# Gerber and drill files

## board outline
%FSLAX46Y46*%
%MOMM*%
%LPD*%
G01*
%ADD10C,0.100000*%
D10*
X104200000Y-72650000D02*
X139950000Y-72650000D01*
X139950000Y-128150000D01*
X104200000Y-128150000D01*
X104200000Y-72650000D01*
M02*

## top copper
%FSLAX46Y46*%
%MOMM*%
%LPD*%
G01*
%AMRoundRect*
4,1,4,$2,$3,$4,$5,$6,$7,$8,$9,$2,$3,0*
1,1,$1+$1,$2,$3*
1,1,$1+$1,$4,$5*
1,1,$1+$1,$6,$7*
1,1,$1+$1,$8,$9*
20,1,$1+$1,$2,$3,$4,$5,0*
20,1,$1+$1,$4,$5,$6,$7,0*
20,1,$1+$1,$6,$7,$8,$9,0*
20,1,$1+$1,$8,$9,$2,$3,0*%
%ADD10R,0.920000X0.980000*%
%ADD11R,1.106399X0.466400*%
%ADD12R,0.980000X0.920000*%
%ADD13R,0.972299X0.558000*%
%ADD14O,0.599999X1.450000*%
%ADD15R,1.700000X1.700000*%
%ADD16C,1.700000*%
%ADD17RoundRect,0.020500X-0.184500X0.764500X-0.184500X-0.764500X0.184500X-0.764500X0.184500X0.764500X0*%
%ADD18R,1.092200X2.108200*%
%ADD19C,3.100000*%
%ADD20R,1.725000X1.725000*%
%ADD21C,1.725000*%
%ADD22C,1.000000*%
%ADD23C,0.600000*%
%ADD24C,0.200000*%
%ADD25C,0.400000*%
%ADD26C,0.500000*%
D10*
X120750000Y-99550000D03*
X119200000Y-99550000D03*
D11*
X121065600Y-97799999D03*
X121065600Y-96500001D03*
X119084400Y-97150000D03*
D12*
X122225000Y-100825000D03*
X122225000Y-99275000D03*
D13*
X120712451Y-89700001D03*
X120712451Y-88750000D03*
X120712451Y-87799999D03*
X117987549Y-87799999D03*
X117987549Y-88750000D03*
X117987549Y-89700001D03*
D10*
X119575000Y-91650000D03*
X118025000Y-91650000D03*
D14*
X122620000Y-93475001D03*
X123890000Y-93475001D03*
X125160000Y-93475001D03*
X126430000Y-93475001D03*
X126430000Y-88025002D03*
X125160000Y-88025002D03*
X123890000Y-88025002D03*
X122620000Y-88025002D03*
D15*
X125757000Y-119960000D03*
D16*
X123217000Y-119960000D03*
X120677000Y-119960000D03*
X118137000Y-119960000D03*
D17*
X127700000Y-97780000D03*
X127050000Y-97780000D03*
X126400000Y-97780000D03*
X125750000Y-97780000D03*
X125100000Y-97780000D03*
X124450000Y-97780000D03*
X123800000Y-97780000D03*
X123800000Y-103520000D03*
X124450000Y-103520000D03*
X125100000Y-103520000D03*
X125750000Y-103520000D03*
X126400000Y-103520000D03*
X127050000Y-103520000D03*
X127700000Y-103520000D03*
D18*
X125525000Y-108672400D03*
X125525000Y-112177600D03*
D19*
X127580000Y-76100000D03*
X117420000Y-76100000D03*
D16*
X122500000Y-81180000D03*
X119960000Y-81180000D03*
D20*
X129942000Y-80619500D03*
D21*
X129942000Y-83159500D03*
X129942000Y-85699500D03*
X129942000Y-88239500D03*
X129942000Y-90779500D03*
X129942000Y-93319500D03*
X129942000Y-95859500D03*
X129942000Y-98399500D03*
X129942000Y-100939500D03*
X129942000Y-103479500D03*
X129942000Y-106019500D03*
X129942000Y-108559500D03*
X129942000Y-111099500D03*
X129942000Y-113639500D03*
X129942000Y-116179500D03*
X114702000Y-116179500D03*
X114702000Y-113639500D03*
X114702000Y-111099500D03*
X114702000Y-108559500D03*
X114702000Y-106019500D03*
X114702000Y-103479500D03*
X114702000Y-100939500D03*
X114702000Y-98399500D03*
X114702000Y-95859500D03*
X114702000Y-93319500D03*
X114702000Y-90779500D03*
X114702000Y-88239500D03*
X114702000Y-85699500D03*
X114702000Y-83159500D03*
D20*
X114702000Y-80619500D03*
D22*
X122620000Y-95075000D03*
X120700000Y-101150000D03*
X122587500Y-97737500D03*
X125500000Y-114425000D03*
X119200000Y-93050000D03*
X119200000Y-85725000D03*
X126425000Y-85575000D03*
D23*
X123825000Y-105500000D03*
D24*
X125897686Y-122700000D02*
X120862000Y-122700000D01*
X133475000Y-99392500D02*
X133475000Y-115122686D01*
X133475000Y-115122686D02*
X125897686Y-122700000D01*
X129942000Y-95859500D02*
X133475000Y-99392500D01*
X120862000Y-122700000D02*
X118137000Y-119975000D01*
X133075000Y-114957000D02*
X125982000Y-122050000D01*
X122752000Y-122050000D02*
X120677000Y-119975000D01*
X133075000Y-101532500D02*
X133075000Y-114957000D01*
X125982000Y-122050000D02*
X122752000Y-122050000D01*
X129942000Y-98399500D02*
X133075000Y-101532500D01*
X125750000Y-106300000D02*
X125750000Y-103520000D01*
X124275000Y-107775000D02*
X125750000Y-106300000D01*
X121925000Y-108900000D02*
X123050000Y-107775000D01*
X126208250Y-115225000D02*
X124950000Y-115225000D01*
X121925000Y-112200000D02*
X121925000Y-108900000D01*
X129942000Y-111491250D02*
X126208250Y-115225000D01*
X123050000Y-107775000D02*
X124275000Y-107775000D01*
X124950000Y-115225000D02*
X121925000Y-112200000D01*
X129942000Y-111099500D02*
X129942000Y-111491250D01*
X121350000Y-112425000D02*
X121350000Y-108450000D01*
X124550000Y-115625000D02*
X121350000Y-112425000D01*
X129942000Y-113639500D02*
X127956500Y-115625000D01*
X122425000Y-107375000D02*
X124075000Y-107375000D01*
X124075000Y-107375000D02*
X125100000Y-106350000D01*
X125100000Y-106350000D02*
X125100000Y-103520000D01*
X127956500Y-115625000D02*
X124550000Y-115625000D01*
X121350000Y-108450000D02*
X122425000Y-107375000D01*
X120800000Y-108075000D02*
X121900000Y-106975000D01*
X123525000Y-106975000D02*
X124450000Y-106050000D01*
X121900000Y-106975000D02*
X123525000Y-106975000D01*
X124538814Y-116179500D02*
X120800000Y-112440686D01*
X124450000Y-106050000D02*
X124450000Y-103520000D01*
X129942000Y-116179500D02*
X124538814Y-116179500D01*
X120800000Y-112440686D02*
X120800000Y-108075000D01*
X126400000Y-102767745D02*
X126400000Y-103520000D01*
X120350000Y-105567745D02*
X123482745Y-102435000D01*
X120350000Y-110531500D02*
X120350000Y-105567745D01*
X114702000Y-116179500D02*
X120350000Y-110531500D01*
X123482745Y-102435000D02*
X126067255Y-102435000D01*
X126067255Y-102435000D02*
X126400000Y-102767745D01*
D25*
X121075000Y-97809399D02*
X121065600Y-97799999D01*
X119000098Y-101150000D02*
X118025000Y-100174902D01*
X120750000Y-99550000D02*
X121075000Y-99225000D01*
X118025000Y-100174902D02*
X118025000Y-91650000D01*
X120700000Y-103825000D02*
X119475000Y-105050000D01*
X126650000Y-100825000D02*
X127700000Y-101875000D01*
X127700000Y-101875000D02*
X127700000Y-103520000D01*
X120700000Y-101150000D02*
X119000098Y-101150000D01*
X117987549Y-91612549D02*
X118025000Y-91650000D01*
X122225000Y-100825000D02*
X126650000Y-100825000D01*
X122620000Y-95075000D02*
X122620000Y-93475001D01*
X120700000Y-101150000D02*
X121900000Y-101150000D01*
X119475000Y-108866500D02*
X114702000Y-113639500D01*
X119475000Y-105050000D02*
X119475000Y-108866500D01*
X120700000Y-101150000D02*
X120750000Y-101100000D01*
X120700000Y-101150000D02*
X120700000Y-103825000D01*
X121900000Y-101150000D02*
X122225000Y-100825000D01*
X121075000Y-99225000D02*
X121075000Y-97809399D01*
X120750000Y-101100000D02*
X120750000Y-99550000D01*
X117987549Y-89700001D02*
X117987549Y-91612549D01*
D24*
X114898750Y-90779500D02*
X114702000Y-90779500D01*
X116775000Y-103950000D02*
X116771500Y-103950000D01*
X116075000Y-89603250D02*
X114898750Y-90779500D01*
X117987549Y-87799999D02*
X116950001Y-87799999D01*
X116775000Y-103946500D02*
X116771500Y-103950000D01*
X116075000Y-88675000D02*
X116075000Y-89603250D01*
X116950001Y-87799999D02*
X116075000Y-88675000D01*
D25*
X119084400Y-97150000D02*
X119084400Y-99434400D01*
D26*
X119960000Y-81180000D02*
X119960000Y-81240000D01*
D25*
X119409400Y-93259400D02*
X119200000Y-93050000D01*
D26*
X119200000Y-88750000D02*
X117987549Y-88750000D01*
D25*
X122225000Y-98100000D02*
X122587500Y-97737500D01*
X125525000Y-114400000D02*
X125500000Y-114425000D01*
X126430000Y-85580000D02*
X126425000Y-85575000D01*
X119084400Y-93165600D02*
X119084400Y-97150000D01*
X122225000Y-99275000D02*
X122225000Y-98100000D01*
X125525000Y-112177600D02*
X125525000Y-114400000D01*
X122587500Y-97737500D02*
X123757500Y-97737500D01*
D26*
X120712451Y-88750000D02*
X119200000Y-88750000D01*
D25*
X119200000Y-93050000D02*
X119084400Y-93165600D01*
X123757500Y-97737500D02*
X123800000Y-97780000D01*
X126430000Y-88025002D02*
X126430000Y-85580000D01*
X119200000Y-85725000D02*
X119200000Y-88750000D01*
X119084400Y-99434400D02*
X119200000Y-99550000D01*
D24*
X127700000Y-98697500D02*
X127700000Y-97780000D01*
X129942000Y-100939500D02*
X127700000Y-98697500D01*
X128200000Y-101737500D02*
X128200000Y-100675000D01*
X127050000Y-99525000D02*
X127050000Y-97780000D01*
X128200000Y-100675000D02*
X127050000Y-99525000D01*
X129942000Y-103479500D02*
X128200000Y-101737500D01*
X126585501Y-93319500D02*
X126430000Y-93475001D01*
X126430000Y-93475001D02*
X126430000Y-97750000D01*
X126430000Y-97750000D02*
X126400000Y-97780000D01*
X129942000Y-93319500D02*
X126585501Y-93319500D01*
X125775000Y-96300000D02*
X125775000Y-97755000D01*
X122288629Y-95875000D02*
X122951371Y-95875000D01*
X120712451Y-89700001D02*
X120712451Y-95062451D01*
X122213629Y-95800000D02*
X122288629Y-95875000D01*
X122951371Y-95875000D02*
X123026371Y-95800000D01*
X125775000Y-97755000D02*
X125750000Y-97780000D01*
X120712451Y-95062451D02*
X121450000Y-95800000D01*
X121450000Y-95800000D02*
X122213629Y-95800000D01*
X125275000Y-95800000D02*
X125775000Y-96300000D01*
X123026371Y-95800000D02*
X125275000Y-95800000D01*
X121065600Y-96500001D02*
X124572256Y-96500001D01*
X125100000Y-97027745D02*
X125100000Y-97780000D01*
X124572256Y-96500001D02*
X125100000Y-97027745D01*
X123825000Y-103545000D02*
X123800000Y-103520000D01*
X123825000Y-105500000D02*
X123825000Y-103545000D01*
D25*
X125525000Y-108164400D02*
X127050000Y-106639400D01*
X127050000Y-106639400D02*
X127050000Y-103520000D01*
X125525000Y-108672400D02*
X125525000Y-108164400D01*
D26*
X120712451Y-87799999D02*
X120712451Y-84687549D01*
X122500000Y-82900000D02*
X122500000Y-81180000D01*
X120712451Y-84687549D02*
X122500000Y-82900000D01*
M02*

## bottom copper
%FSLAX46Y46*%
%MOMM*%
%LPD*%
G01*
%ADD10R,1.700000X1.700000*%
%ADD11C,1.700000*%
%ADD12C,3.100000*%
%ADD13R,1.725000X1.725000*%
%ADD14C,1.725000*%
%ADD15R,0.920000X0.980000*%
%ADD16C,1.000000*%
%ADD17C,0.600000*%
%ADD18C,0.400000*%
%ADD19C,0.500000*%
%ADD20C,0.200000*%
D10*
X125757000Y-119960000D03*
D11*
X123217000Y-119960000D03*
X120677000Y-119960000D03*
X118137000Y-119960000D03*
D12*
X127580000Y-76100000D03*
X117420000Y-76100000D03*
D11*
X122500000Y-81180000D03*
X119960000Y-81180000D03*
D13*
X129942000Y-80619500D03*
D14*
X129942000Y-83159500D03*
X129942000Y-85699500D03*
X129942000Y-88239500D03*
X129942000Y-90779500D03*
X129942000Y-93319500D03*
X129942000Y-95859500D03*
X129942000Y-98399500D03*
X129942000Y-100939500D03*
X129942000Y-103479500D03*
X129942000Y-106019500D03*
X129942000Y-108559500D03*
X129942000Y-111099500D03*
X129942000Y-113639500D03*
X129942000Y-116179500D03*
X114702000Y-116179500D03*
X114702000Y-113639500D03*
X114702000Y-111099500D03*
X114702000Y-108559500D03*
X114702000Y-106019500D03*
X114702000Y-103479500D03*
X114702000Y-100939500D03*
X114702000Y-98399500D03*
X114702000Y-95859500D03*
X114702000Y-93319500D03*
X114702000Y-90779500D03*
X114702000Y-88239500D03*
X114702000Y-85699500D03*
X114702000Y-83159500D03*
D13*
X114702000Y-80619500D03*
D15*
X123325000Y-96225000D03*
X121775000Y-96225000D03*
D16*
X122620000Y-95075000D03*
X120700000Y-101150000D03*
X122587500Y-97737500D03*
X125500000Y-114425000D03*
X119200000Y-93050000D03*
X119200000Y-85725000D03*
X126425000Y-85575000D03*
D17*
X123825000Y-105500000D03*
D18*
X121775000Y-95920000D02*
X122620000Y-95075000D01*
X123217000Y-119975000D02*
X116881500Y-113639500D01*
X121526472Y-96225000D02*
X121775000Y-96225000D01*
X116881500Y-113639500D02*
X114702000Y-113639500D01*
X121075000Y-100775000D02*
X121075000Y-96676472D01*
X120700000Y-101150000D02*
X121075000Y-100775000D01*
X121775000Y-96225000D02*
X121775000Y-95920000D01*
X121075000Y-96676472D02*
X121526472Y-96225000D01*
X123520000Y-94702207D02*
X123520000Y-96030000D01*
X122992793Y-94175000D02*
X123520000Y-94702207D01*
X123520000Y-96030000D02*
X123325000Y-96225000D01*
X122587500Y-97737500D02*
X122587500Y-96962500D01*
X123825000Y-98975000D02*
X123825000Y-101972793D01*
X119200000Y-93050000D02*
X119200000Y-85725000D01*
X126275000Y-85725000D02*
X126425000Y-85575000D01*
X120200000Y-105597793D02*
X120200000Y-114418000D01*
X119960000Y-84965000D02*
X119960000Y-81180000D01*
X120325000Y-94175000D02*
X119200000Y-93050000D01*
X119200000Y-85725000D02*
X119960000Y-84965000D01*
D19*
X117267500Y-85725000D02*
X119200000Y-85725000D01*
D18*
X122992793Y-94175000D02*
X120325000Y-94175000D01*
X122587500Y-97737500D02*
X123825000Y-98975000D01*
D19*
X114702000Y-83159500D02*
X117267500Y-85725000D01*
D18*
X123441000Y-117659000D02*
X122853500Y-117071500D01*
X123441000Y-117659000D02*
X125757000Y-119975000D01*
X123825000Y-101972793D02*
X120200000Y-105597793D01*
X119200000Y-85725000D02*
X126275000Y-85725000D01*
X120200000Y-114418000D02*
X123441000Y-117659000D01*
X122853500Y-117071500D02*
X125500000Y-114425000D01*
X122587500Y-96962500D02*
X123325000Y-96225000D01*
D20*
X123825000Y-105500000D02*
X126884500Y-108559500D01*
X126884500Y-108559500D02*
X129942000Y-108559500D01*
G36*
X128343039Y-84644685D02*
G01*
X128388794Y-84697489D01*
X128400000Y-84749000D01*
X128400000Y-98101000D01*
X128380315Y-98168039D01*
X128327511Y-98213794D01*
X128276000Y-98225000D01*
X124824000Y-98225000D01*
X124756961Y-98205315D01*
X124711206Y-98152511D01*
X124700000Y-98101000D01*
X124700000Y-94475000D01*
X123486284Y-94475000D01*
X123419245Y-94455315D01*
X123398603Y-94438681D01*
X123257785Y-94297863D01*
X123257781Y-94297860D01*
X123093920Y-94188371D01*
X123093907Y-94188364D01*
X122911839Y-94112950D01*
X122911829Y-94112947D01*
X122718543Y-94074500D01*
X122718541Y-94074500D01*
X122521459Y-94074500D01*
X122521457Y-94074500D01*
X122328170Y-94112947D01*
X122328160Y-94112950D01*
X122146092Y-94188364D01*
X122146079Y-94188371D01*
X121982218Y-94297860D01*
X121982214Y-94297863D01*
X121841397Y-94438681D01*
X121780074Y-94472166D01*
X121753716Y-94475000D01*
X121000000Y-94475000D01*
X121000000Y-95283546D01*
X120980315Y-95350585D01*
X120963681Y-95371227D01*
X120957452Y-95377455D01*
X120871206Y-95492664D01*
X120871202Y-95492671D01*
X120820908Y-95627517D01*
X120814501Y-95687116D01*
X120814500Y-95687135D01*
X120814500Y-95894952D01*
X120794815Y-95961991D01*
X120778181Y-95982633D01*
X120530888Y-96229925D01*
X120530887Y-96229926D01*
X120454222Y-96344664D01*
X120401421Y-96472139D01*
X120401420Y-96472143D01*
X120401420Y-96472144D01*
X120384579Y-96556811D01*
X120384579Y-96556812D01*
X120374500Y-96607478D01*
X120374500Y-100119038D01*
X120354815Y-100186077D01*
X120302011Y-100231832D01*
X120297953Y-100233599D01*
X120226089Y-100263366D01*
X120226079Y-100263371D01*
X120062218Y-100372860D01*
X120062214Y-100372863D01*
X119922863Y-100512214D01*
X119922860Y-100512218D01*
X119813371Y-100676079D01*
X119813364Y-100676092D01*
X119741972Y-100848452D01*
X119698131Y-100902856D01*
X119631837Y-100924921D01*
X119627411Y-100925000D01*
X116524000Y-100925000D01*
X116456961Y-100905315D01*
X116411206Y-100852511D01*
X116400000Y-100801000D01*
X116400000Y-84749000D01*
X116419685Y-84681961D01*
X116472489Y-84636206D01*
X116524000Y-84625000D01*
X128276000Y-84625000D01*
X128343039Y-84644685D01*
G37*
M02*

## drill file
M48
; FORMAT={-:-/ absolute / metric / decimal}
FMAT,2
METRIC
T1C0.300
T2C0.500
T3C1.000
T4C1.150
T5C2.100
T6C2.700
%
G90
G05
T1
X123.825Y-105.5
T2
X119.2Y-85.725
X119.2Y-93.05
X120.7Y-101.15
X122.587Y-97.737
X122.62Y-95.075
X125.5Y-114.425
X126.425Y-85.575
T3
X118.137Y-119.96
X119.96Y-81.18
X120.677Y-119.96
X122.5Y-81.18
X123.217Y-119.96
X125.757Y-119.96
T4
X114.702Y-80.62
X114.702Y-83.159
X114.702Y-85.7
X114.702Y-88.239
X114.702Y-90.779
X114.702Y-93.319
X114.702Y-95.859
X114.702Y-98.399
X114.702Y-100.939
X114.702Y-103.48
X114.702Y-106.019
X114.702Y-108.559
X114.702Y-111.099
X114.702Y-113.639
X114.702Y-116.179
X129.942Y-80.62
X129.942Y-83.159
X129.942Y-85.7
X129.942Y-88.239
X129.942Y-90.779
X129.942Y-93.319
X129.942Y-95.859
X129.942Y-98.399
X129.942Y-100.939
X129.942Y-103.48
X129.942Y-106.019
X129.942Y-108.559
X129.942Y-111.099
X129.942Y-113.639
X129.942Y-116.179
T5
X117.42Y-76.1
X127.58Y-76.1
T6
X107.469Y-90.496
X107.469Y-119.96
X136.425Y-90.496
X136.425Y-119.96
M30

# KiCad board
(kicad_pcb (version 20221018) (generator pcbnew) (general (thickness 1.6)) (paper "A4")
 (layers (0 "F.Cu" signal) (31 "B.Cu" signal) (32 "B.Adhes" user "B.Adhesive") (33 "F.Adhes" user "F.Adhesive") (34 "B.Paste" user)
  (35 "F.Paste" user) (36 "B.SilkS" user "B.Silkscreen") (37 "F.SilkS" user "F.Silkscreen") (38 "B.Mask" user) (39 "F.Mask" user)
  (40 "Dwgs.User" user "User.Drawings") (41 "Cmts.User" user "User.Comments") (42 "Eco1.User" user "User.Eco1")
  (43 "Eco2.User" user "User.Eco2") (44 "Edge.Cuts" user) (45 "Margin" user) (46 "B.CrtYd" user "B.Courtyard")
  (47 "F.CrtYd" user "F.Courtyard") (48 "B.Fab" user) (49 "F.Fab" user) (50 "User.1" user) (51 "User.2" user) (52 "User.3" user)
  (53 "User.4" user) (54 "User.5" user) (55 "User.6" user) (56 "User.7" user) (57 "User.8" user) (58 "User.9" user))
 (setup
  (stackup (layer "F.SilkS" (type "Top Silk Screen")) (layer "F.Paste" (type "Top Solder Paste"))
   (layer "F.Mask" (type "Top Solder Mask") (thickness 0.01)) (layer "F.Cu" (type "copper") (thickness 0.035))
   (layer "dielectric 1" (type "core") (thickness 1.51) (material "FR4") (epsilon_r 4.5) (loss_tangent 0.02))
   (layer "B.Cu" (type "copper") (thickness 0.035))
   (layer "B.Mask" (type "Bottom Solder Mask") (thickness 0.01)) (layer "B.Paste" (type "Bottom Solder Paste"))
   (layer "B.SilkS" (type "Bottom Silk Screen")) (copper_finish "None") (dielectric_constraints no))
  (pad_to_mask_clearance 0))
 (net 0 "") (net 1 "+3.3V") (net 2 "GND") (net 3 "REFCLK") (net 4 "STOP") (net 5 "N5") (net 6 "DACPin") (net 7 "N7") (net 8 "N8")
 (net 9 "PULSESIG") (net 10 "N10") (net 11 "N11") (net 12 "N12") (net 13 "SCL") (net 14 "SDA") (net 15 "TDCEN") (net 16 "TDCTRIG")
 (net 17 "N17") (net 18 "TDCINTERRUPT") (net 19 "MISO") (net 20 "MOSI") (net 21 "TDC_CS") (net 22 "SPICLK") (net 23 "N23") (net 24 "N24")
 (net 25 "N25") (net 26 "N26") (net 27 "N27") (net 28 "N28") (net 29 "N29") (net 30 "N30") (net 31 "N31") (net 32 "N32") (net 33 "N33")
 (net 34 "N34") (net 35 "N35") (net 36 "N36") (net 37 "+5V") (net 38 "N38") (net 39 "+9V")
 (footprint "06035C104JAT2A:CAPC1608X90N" (layer "F.Cu") (at 119.975 99.55 180)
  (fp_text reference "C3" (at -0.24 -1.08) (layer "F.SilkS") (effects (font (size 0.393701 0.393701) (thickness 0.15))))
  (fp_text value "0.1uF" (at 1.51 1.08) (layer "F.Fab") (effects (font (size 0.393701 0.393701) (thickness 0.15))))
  (pad "1" smd rect (at -0.775 0 180) (size 0.92 0.98) (layers "F.Cu" "F.Paste" "F.Mask") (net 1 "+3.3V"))
  (pad "2" smd rect (at 0.775 0 180) (size 0.92 0.98) (layers "F.Cu" "F.Paste" "F.Mask") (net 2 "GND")))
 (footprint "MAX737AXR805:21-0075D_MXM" (layer "F.Cu") (at 120.075 97.15 90)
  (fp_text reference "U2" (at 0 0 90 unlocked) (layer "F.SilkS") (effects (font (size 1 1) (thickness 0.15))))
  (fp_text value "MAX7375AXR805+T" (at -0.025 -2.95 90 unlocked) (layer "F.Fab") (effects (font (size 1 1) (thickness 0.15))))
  (pad "1" smd rect (at -0.649999 0.9906 90) (size 0.4664 1.106399) (layers "F.Cu" "F.Paste" "F.Mask") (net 1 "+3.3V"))
  (pad "2" smd rect (at 0.649999 0.9906 90) (size 0.4664 1.106399) (layers "F.Cu" "F.Paste" "F.Mask") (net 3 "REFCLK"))
  (pad "3" smd rect (at 0 -0.9906 90) (size 0.4664 1.106399) (layers "F.Cu" "F.Paste" "F.Mask") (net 2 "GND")))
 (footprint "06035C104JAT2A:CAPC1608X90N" (layer "F.Cu") (at 122.225 100.05 90)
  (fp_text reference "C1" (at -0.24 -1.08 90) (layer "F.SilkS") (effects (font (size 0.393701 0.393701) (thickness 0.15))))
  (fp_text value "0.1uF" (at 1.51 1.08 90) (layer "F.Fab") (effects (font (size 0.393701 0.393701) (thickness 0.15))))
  (pad "1" smd rect (at -0.775 0 90) (size 0.92 0.98) (layers "F.Cu" "F.Paste" "F.Mask") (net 1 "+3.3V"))
  (pad "2" smd rect (at 0.775 0 90) (size 0.92 0.98) (layers "F.Cu" "F.Paste" "F.Mask") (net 2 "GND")))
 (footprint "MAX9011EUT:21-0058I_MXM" (layer "F.Cu") (at 119.35 88.75 180)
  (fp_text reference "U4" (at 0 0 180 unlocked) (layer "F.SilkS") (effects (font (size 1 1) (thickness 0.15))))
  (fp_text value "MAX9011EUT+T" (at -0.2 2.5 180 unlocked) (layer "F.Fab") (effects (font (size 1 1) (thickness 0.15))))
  (pad "1" smd rect (at -1.362451 -0.950001 180) (size 0.972299 0.558) (layers "F.Cu" "F.Paste" "F.Mask") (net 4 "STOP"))
  (pad "2" smd rect (at -1.362451 0 180) (size 0.972299 0.558) (layers "F.Cu" "F.Paste" "F.Mask") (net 2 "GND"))
  (pad "3" smd rect (at -1.362451 0.950001 180) (size 0.972299 0.558) (layers "F.Cu" "F.Paste" "F.Mask") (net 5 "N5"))
  (pad "4" smd rect (at 1.362451 0.950001 180) (size 0.972299 0.558) (layers "F.Cu" "F.Paste" "F.Mask") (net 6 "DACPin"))
  (pad "5" smd rect (at 1.362451 0 180) (size 0.972299 0.558) (layers "F.Cu" "F.Paste" "F.Mask") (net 2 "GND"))
  (pad "6" smd rect (at 1.362451 -0.950001 180) (size 0.972299 0.558) (layers "F.Cu" "F.Paste" "F.Mask") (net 1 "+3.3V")))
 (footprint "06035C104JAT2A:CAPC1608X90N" (layer "F.Cu") (at 118.8 91.65 180)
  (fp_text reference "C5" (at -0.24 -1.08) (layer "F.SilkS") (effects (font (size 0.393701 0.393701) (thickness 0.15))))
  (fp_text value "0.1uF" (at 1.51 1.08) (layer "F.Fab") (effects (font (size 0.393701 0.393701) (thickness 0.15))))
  (pad "1" smd rect (at -0.775 0 180) (size 0.92 0.98) (layers "F.Cu" "F.Paste" "F.Mask") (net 2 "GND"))
  (pad "2" smd rect (at 0.775 0 180) (size 0.92 0.98) (layers "F.Cu" "F.Paste" "F.Mask") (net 1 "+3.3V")))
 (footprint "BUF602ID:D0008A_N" (layer "F.Cu") (at 124.525 90.75 90)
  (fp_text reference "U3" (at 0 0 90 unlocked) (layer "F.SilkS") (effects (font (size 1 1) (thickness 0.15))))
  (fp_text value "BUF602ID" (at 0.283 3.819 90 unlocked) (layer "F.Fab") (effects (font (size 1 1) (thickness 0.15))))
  (pad "1" smd oval (at -2.725001 -1.905 180) (size 0.599999 1.45) (layers "F.Cu" "F.Paste" "F.Mask") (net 1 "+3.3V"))
  (pad "2" smd oval (at -2.725001 -0.635 180) (size 0.599999 1.45) (layers "F.Cu" "F.Paste" "F.Mask") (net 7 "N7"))
  (pad "3" smd oval (at -2.725001 0.635 180) (size 0.599999 1.45) (layers "F.Cu" "F.Paste" "F.Mask") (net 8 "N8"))
  (pad "4" smd oval (at -2.725001 1.905 180) (size 0.599999 1.45) (layers "F.Cu" "F.Paste" "F.Mask") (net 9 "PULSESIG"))
  (pad "5" smd oval (at 2.724998 1.905 180) (size 0.599999 1.45) (layers "F.Cu" "F.Paste" "F.Mask") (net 2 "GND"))
  (pad "6" smd oval (at 2.724998 0.635 180) (size 0.599999 1.45) (layers "F.Cu" "F.Paste" "F.Mask") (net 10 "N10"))
  (pad "7" smd oval (at 2.724998 -0.635 180) (size 0.599999 1.45) (layers "F.Cu" "F.Paste" "F.Mask") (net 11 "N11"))
  (pad "8" smd oval (at 2.724998 -1.905 180) (size 0.599999 1.45) (layers "F.Cu" "F.Paste" "F.Mask") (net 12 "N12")))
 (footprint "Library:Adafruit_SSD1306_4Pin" (layer "F.Cu") (at 130.837 119.96 180)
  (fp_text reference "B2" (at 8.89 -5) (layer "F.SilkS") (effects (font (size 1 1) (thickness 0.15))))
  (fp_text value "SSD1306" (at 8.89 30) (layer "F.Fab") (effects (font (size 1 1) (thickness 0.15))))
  (pad "" np_thru_hole circle (at -5.588 0 180) (size 2.7 2.7) (drill 2.7) (layers "*.Cu" "*.Mask"))
  (pad "" np_thru_hole circle (at -5.588 29.464 180) (size 2.7 2.7) (drill 2.7) (layers "*.Cu" "*.Mask"))
  (pad "" np_thru_hole circle (at 23.368 0 180) (size 2.7 2.7) (drill 2.7) (layers "*.Cu" "*.Mask"))
  (pad "" np_thru_hole circle (at 23.368 29.464 180) (size 2.7 2.7) (drill 2.7) (layers "*.Cu" "*.Mask"))
  (pad "1" thru_hole rect (at 5.08 0 180) (size 1.7 1.7) (drill 1) (layers "*.Cu" "*.Mask") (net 2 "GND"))
  (pad "2" thru_hole circle (at 7.62 0 180) (size 1.7 1.7) (drill 1) (layers "*.Cu" "*.Mask") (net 1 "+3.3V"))
  (pad "3" thru_hole circle (at 10.16 0 180) (size 1.7 1.7) (drill 1) (layers "*.Cu" "*.Mask") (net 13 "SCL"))
  (pad "4" thru_hole circle (at 12.7 0 180) (size 1.7 1.7) (drill 1) (layers "*.Cu" "*.Mask") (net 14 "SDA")))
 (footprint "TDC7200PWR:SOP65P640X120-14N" (layer "F.Cu") (at 125.75 100.65 -90)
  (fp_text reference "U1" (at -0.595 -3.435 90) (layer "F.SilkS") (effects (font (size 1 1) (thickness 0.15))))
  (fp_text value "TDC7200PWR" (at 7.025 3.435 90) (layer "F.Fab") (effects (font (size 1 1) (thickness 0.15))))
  (pad "1" smd roundrect (at -2.87 -1.95 270) (size 1.57 0.41) (layers "F.Cu" "F.Paste" "F.Mask") (roundrect_rratio 0.05) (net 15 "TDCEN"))
  (pad "2" smd roundrect (at -2.87 -1.3 270) (size 1.57 0.41) (layers "F.Cu" "F.Paste" "F.Mask") (roundrect_rratio 0.05) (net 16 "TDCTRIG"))
  (pad "3" smd roundrect (at -2.87 -0.65 270) (size 1.57 0.41) (layers "F.Cu" "F.Paste" "F.Mask") (roundrect_rratio 0.05) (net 9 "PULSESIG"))
  (pad "4" smd roundrect (at -2.87 0 270) (size 1.57 0.41) (layers "F.Cu" "F.Paste" "F.Mask") (roundrect_rratio 0.05) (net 4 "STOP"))
  (pad "5" smd roundrect (at -2.87 0.65 270) (size 1.57 0.41) (layers "F.Cu" "F.Paste" "F.Mask") (roundrect_rratio 0.05) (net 3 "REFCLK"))
  (pad "6" smd roundrect (at -2.87 1.3 270) (size 1.57 0.41) (layers "F.Cu" "F.Paste" "F.Mask") (roundrect_rratio 0.05) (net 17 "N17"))
  (pad "7" smd roundrect (at -2.87 1.95 270) (size 1.57 0.41) (layers "F.Cu" "F.Paste" "F.Mask") (roundrect_rratio 0.05) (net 2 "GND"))
  (pad "8" smd roundrect (at 2.87 1.95 270) (size 1.57 0.41) (layers "F.Cu" "F.Paste" "F.Mask") (roundrect_rratio 0.05)
   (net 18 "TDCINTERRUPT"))
  (pad "9" smd roundrect (at 2.87 1.3 270) (size 1.57 0.41) (layers "F.Cu" "F.Paste" "F.Mask") (roundrect_rratio 0.05) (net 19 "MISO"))
  (pad "10" smd roundrect (at 2.87 0.65 270) (size 1.57 0.41) (layers "F.Cu" "F.Paste" "F.Mask") (roundrect_rratio 0.05) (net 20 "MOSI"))
  (pad "11" smd roundrect (at 2.87 0 270) (size 1.57 0.41) (layers "F.Cu" "F.Paste" "F.Mask") (roundrect_rratio 0.05) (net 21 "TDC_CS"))
  (pad "12" smd roundrect (at 2.87 -0.65 270) (size 1.57 0.41) (layers "F.Cu" "F.Paste" "F.Mask") (roundrect_rratio 0.05) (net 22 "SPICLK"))
  (pad "13" smd roundrect (at 2.87 -1.3 270) (size 1.57 0.41) (layers "F.Cu" "F.Paste" "F.Mask") (roundrect_rratio 0.05) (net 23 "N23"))
  (pad "14" smd roundrect (at 2.87 -1.95 270) (size 1.57 0.41) (layers "F.Cu" "F.Paste" "F.Mask") (roundrect_rratio 0.05) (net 1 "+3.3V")))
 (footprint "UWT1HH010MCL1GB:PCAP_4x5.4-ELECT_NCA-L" (layer "F.Cu") (at 125.525 110.425 -90)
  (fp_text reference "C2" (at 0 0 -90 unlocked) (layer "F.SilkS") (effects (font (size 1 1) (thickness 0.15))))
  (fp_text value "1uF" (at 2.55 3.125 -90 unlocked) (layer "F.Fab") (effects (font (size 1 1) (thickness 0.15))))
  (pad "1" smd rect (at -1.7526 0 270) (size 2.1082 1.0922) (layers "F.Cu" "F.Paste" "F.Mask") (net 23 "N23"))
  (pad "2" smd rect (at 1.7526 0 270) (size 2.1082 1.0922) (layers "F.Cu" "F.Paste" "F.Mask") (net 2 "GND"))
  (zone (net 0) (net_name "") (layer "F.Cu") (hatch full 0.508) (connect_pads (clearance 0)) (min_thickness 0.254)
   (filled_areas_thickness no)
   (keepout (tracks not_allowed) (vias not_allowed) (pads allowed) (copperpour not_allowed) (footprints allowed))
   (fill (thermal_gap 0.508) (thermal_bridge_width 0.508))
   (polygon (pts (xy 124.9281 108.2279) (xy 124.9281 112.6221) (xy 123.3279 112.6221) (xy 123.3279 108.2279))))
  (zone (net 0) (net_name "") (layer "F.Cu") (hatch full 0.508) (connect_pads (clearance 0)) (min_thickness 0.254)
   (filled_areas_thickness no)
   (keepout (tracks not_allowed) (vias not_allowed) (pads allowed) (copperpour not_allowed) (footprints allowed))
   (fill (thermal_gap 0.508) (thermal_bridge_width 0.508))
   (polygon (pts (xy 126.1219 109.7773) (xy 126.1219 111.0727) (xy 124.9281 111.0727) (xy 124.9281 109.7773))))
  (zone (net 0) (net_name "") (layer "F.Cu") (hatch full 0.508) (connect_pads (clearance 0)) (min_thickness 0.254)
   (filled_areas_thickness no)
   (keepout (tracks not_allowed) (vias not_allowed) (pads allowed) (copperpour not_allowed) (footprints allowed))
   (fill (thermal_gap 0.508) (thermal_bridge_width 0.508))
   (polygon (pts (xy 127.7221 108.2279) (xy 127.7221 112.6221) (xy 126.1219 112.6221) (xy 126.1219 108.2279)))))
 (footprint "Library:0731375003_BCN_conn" (layer "F.Cu") (at 122.5 76.1 180)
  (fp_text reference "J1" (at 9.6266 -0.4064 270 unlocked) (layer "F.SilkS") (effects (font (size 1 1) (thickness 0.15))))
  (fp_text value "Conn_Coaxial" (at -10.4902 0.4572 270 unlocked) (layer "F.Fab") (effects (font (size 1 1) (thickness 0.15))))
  (pad "" thru_hole circle (at -5.08 0 180) (size 3.1 3.1) (drill 2.1) (layers "*.Cu" "*.Mask"))
  (pad "" thru_hole circle (at 5.08 0 180) (size 3.1 3.1) (drill 2.1) (layers "*.Cu" "*.Mask"))
  (pad "1" thru_hole circle (at 0 -5.08 180) (size 1.7 1.7) (drill 1) (layers "*.Cu" "*.Mask" "Eco2.User") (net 5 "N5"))
  (pad "2" thru_hole circle (at 2.54 -5.08 180) (size 1.7 1.7) (drill 1) (layers "*.Cu" "*.Mask") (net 2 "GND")))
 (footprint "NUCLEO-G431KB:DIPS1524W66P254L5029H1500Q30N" (layer "B.Cu") (at 122.322 98.3995 180)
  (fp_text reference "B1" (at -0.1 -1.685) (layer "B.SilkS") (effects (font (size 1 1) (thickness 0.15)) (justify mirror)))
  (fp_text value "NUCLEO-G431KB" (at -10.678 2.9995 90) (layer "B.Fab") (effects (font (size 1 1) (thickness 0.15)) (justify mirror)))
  (pad "1" thru_hole rect (at -7.62 17.78 180) (size 1.725 1.725) (drill 1.15) (layers "*.Cu" "*.Mask") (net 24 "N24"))
  (pad "2" thru_hole circle (at -7.62 15.24 180) (size 1.725 1.725) (drill 1.15) (layers "*.Cu" "*.Mask") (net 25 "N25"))
  (pad "3" thru_hole circle (at -7.62 12.7 180) (size 1.725 1.725) (drill 1.15) (layers "*.Cu" "*.Mask") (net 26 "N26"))
  (pad "4" thru_hole circle (at -7.62 10.16 180) (size 1.725 1.725) (drill 1.15) (layers "*.Cu" "*.Mask") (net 2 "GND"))
  (pad "5" thru_hole circle (at -7.62 7.62 180) (size 1.725 1.725) (drill 1.15) (layers "*.Cu" "*.Mask") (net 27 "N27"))
  (pad "6" thru_hole circle (at -7.62 5.08 180) (size 1.725 1.725) (drill 1.15) (layers "*.Cu" "*.Mask") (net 9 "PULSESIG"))
  (pad "7" thru_hole circle (at -7.62 2.54 180) (size 1.725 1.725) (drill 1.15) (layers "*.Cu" "*.Mask") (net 14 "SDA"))
  (pad "8" thru_hole circle (at -7.62 0 180) (size 1.725 1.725) (drill 1.15) (layers "*.Cu" "*.Mask") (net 13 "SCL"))
  (pad "9" thru_hole circle (at -7.62 -2.54 180) (size 1.725 1.725) (drill 1.15) (layers "*.Cu" "*.Mask") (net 15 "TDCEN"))
  (pad "10" thru_hole circle (at -7.62 -5.08 180) (size 1.725 1.725) (drill 1.15) (layers "*.Cu" "*.Mask") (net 16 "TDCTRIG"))
  (pad "11" thru_hole circle (at -7.62 -7.62 180) (size 1.725 1.725) (drill 1.15) (layers "*.Cu" "*.Mask") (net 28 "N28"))
  (pad "12" thru_hole circle (at -7.62 -10.16 180) (size 1.725 1.725) (drill 1.15) (layers "*.Cu" "*.Mask") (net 18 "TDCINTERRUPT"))
  (pad "13" thru_hole circle (at -7.62 -12.7 180) (size 1.725 1.725) (drill 1.15) (layers "*.Cu" "*.Mask") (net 21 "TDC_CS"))
  (pad "14" thru_hole circle (at -7.62 -15.24 180) (size 1.725 1.725) (drill 1.15) (layers "*.Cu" "*.Mask") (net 20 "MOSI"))
  (pad "15" thru_hole circle (at -7.62 -17.78 180) (size 1.725 1.725) (drill 1.15) (layers "*.Cu" "*.Mask") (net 19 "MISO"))
  (pad "16" thru_hole circle (at 7.62 -17.78 180) (size 1.725 1.725) (drill 1.15) (layers "*.Cu" "*.Mask") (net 22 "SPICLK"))
  (pad "17" thru_hole circle (at 7.62 -15.24 180) (size 1.725 1.725) (drill 1.15) (layers "*.Cu" "*.Mask") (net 1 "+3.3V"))
  (pad "18" thru_hole circle (at 7.62 -12.7 180) (size 1.725 1.725) (drill 1.15) (layers "*.Cu" "*.Mask") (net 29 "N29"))
  (pad "19" thru_hole circle (at 7.62 -10.16 180) (size 1.725 1.725) (drill 1.15) (layers "*.Cu" "*.Mask") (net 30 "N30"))
  (pad "20" thru_hole circle (at 7.62 -7.62 180) (size 1.725 1.725) (drill 1.15) (layers "*.Cu" "*.Mask") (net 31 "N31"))
  (pad "21" thru_hole circle (at 7.62 -5.08 180) (size 1.725 1.725) (drill 1.15) (layers "*.Cu" "*.Mask") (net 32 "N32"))
  (pad "22" thru_hole circle (at 7.62 -2.54 180) (size 1.725 1.725) (drill 1.15) (layers "*.Cu" "*.Mask") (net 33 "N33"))
  (pad "23" thru_hole circle (at 7.62 0 180) (size 1.725 1.725) (drill 1.15) (layers "*.Cu" "*.Mask") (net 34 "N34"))
  (pad "24" thru_hole circle (at 7.62 2.54 180) (size 1.725 1.725) (drill 1.15) (layers "*.Cu" "*.Mask") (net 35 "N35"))
  (pad "25" thru_hole circle (at 7.62 5.08 180) (size 1.725 1.725) (drill 1.15) (layers "*.Cu" "*.Mask") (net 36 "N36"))
  (pad "26" thru_hole circle (at 7.62 7.62 180) (size 1.725 1.725) (drill 1.15) (layers "*.Cu" "*.Mask") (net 6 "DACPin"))
  (pad "27" thru_hole circle (at 7.62 10.16 180) (size 1.725 1.725) (drill 1.15) (layers "*.Cu" "*.Mask") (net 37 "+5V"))
  (pad "28" thru_hole circle (at 7.62 12.7 180) (size 1.725 1.725) (drill 1.15) (layers "*.Cu" "*.Mask") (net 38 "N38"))
  (pad "29" thru_hole circle (at 7.62 15.24 180) (size 1.725 1.725) (drill 1.15) (layers "*.Cu" "*.Mask") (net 2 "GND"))
  (pad "30" thru_hole rect (at 7.62 17.78 180) (size 1.725 1.725) (drill 1.15) (layers "*.Cu" "*.Mask") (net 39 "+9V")))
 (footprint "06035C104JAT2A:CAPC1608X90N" (layer "B.Cu") (at 122.55 96.225 180)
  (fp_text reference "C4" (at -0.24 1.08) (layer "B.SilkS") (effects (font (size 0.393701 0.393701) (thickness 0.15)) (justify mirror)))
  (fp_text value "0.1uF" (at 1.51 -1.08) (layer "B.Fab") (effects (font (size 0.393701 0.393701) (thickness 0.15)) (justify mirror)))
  (pad "1" smd rect (at -0.775 0 180) (size 0.92 0.98) (layers "B.Cu" "B.Paste" "B.Mask") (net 2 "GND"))
  (pad "2" smd rect (at 0.775 0 180) (size 0.92 0.98) (layers "B.Cu" "B.Paste" "B.Mask") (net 1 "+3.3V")))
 (gr_rect (start 104.2 72.65) (end 139.95 128.15) (stroke (width 0.1) (type default)) (fill none) (layer "Edge.Cuts"))
 (segment (start 125.897686 122.7) (end 120.862 122.7) (width 0.2) (layer "F.Cu") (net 14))
 (segment (start 133.475 99.3925) (end 133.475 115.122686) (width 0.2) (layer "F.Cu") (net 14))
 (segment (start 133.475 115.122686) (end 125.897686 122.7) (width 0.2) (layer "F.Cu") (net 14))
 (segment (start 129.942 95.8595) (end 133.475 99.3925) (width 0.2) (layer "F.Cu") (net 14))
 (segment (start 120.862 122.7) (end 118.137 119.975) (width 0.2) (layer "F.Cu") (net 14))
 (segment (start 133.075 114.957) (end 125.982 122.05) (width 0.2) (layer "F.Cu") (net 13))
 (segment (start 122.752 122.05) (end 120.677 119.975) (width 0.2) (layer "F.Cu") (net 13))
 (segment (start 133.075 101.5325) (end 133.075 114.957) (width 0.2) (layer "F.Cu") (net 13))
 (segment (start 125.982 122.05) (end 122.752 122.05) (width 0.2) (layer "F.Cu") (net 13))
 (segment (start 129.942 98.3995) (end 133.075 101.5325) (width 0.2) (layer "F.Cu") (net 13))
 (segment (start 125.75 106.3) (end 125.75 103.52) (width 0.2) (layer "F.Cu") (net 21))
 (segment (start 124.275 107.775) (end 125.75 106.3) (width 0.2) (layer "F.Cu") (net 21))
 (segment (start 121.925 108.9) (end 123.05 107.775) (width 0.2) (layer "F.Cu") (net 21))
 (segment (start 126.20825 115.225) (end 124.95 115.225) (width 0.2) (layer "F.Cu") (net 21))
 (segment (start 121.925 112.2) (end 121.925 108.9) (width 0.2) (layer "F.Cu") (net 21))
 (segment (start 129.942 111.49125) (end 126.20825 115.225) (width 0.2) (layer "F.Cu") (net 21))
 (segment (start 123.05 107.775) (end 124.275 107.775) (width 0.2) (layer "F.Cu") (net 21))
 (segment (start 124.95 115.225) (end 121.925 112.2) (width 0.2) (layer "F.Cu") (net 21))
 (segment (start 129.942 111.0995) (end 129.942 111.49125) (width 0.2) (layer "F.Cu") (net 21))
 (segment (start 121.35 112.425) (end 121.35 108.45) (width 0.2) (layer "F.Cu") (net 20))
 (segment (start 124.55 115.625) (end 121.35 112.425) (width 0.2) (layer "F.Cu") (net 20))
 (segment (start 129.942 113.6395) (end 127.9565 115.625) (width 0.2) (layer "F.Cu") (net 20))
 (segment (start 122.425 107.375) (end 124.075 107.375) (width 0.2) (layer "F.Cu") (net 20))
 (segment (start 124.075 107.375) (end 125.1 106.35) (width 0.2) (layer "F.Cu") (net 20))
 (segment (start 125.1 106.35) (end 125.1 103.52) (width 0.2) (layer "F.Cu") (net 20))
 (segment (start 127.9565 115.625) (end 124.55 115.625) (width 0.2) (layer "F.Cu") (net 20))
 (segment (start 121.35 108.45) (end 122.425 107.375) (width 0.2) (layer "F.Cu") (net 20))
 (segment (start 120.8 108.075) (end 121.9 106.975) (width 0.2) (layer "F.Cu") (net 19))
 (segment (start 123.525 106.975) (end 124.45 106.05) (width 0.2) (layer "F.Cu") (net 19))
 (segment (start 121.9 106.975) (end 123.525 106.975) (width 0.2) (layer "F.Cu") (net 19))
 (segment (start 124.538814 116.1795) (end 120.8 112.440686) (width 0.2) (layer "F.Cu") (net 19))
 (segment (start 124.45 106.05) (end 124.45 103.52) (width 0.2) (layer "F.Cu") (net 19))
 (segment (start 129.942 116.1795) (end 124.538814 116.1795) (width 0.2) (layer "F.Cu") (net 19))
 (segment (start 120.8 112.440686) (end 120.8 108.075) (width 0.2) (layer "F.Cu") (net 19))
 (segment (start 126.4 102.767745) (end 126.4 103.52) (width 0.2) (layer "F.Cu") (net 22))
 (segment (start 120.35 105.567745) (end 123.482745 102.435) (width 0.2) (layer "F.Cu") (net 22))
 (segment (start 120.35 110.5315) (end 120.35 105.567745) (width 0.2) (layer "F.Cu") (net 22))
 (segment (start 114.702 116.1795) (end 120.35 110.5315) (width 0.2) (layer "F.Cu") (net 22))
 (segment (start 123.482745 102.435) (end 126.067255 102.435) (width 0.2) (layer "F.Cu") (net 22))
 (segment (start 126.067255 102.435) (end 126.4 102.767745) (width 0.2) (layer "F.Cu") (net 22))
 (segment (start 121.075 97.809399) (end 121.0656 97.799999) (width 0.4) (layer "F.Cu") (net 1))
 (segment (start 119.000098 101.15) (end 118.025 100.174902) (width 0.4) (layer "F.Cu") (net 1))
 (segment (start 120.75 99.55) (end 121.075 99.225) (width 0.4) (layer "F.Cu") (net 1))
 (segment (start 118.025 100.174902) (end 118.025 91.65) (width 0.4) (layer "F.Cu") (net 1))
 (segment (start 120.7 103.825) (end 119.475 105.05) (width 0.4) (layer "F.Cu") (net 1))
 (segment (start 126.65 100.825) (end 127.7 101.875) (width 0.4) (layer "F.Cu") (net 1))
 (segment (start 127.7 101.875) (end 127.7 103.52) (width 0.4) (layer "F.Cu") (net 1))
 (segment (start 120.7 101.15) (end 119.000098 101.15) (width 0.4) (layer "F.Cu") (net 1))
 (segment (start 117.987549 91.612549) (end 118.025 91.65) (width 0.4) (layer "F.Cu") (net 1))
 (segment (start 122.225 100.825) (end 126.65 100.825) (width 0.4) (layer "F.Cu") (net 1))
 (segment (start 122.62 95.075) (end 122.62 93.475001) (width 0.4) (layer "F.Cu") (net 1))
 (segment (start 120.7 101.15) (end 121.9 101.15) (width 0.4) (layer "F.Cu") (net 1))
 (segment (start 119.475 108.8665) (end 114.702 113.6395) (width 0.4) (layer "F.Cu") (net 1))
 (segment (start 119.475 105.05) (end 119.475 108.8665) (width 0.4) (layer "F.Cu") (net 1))
 (segment (start 120.7 101.15) (end 120.75 101.1) (width 0.4) (layer "F.Cu") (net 1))
 (segment (start 120.7 101.15) (end 120.7 103.825) (width 0.4) (layer "F.Cu") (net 1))
 (segment (start 121.9 101.15) (end 122.225 100.825) (width 0.4) (layer "F.Cu") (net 1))
 (segment (start 121.075 99.225) (end 121.075 97.809399) (width 0.4) (layer "F.Cu") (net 1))
 (segment (start 120.75 101.1) (end 120.75 99.55) (width 0.4) (layer "F.Cu") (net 1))
 (segment (start 117.987549 89.700001) (end 117.987549 91.612549) (width 0.4) (layer "F.Cu") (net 1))
 (via (at 122.62 95.075) (size 1) (drill 0.5) (layers "F.Cu" "B.Cu") (free) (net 1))
 (via (at 120.7 101.15) (size 1) (drill 0.5) (layers "F.Cu" "B.Cu") (free) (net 1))
 (segment (start 121.775 95.92) (end 122.62 95.075) (width 0.4) (layer "B.Cu") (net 1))
 (segment (start 123.217 119.975) (end 116.8815 113.6395) (width 0.4) (layer "B.Cu") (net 1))
 (segment (start 121.526472 96.225) (end 121.775 96.225) (width 0.4) (layer "B.Cu") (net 1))
 (segment (start 116.8815 113.6395) (end 114.702 113.6395) (width 0.4) (layer "B.Cu") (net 1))
 (segment (start 121.075 100.775) (end 121.075 96.676472) (width 0.4) (layer "B.Cu") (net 1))
 (segment (start 120.7 101.15) (end 121.075 100.775) (width 0.4) (layer "B.Cu") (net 1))
 (segment (start 121.775 96.225) (end 121.775 95.92) (width 0.4) (layer "B.Cu") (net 1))
 (segment (start 121.075 96.676472) (end 121.526472 96.225) (width 0.4) (layer "B.Cu") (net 1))
 (segment (start 114.89875 90.7795) (end 114.702 90.7795) (width 0.2) (layer "F.Cu") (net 6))
 (segment (start 116.775 103.95) (end 116.7715 103.95) (width 0.2) (layer "F.Cu") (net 6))
 (segment (start 116.075 89.60325) (end 114.89875 90.7795) (width 0.2) (layer "F.Cu") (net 6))
 (segment (start 117.987549 87.799999) (end 116.950001 87.799999) (width 0.2) (layer "F.Cu") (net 6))
 (segment (start 116.775 103.9465) (end 116.7715 103.95) (width 0.2) (layer "F.Cu") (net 6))
 (segment (start 116.075 88.675) (end 116.075 89.60325) (width 0.2) (layer "F.Cu") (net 6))
 (segment (start 116.950001 87.799999) (end 116.075 88.675) (width 0.2) (layer "F.Cu") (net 6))
 (segment (start 119.0844 97.15) (end 119.0844 99.4344) (width 0.4) (layer "F.Cu") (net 2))
 (segment (start 119.96 81.18) (end 119.96 81.24) (width 0.5) (layer "F.Cu") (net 2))
 (segment (start 119.4094 93.2594) (end 119.2 93.05) (width 0.4) (layer "F.Cu") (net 2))
 (segment (start 119.2 88.75) (end 117.987549 88.75) (width 0.5) (layer "F.Cu") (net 2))
 (segment (start 122.225 98.1) (end 122.5875 97.7375) (width 0.4) (layer "F.Cu") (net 2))
 (segment (start 125.525 114.4) (end 125.5 114.425) (width 0.4) (layer "F.Cu") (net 2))
 (segment (start 126.43 85.58) (end 126.425 85.575) (width 0.4) (layer "F.Cu") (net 2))
 (segment (start 119.0844 93.1656) (end 119.0844 97.15) (width 0.4) (layer "F.Cu") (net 2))
 (segment (start 122.225 99.275) (end 122.225 98.1) (width 0.4) (layer "F.Cu") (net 2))
 (segment (start 125.525 112.1776) (end 125.525 114.4) (width 0.4) (layer "F.Cu") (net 2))
 (segment (start 122.5875 97.7375) (end 123.7575 97.7375) (width 0.4) (layer "F.Cu") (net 2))
 (segment (start 120.712451 88.75) (end 119.2 88.75) (width 0.5) (layer "F.Cu") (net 2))
 (segment (start 119.2 93.05) (end 119.0844 93.1656) (width 0.4) (layer "F.Cu") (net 2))
 (segment (start 123.7575 97.7375) (end 123.8 97.78) (width 0.4) (layer "F.Cu") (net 2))
 (segment (start 126.43 88.025002) (end 126.43 85.58) (width 0.4) (layer "F.Cu") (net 2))
 (segment (start 119.2 85.725) (end 119.2 88.75) (width 0.4) (layer "F.Cu") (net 2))
 (segment (start 119.0844 99.4344) (end 119.2 99.55) (width 0.4) (layer "F.Cu") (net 2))
 (via (at 122.5875 97.7375) (size 1) (drill 0.5) (layers "F.Cu" "B.Cu") (free) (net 2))
 (via (at 125.5 114.425) (size 1) (drill 0.5) (layers "F.Cu" "B.Cu") (free) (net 2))
 (via (at 119.2 93.05) (size 1) (drill 0.5) (layers "F.Cu" "B.Cu") (free) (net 2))
 (via (at 119.2 85.725) (size 1) (drill 0.5) (layers "F.Cu" "B.Cu") (free) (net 2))
 (via (at 126.425 85.575) (size 1) (drill 0.5) (layers "F.Cu" "B.Cu") (free) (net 2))
 (segment (start 123.52 94.702207) (end 123.52 96.03) (width 0.4) (layer "B.Cu") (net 2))
 (segment (start 122.992793 94.175) (end 123.52 94.702207) (width 0.4) (layer "B.Cu") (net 2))
 (segment (start 123.52 96.03) (end 123.325 96.225) (width 0.4) (layer "B.Cu") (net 2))
 (segment (start 122.5875 97.7375) (end 122.5875 96.9625) (width 0.4) (layer "B.Cu") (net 2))
 (segment (start 123.825 98.975) (end 123.825 101.972793) (width 0.4) (layer "B.Cu") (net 2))
 (segment (start 119.2 93.05) (end 119.2 85.725) (width 0.4) (layer "B.Cu") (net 2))
 (segment (start 126.275 85.725) (end 126.425 85.575) (width 0.4) (layer "B.Cu") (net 2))
 (segment (start 120.2 105.597793) (end 120.2 114.418) (width 0.4) (layer "B.Cu") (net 2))
 (segment (start 119.96 84.965) (end 119.96 81.18) (width 0.4) (layer "B.Cu") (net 2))
 (segment (start 120.325 94.175) (end 119.2 93.05) (width 0.4) (layer "B.Cu") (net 2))
 (segment (start 119.2 85.725) (end 119.96 84.965) (width 0.4) (layer "B.Cu") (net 2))
 (segment (start 117.2675 85.725) (end 119.2 85.725) (width 0.5) (layer "B.Cu") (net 2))
 (segment (start 122.992793 94.175) (end 120.325 94.175) (width 0.4) (layer "B.Cu") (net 2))
 (segment (start 122.5875 97.7375) (end 123.825 98.975) (width 0.4) (layer "B.Cu") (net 2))
 (segment (start 114.702 83.1595) (end 117.2675 85.725) (width 0.5) (layer "B.Cu") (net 2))
 (segment (start 123.441 117.659) (end 122.8535 117.0715) (width 0.4) (layer "B.Cu") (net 2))
 (segment (start 123.441 117.659) (end 125.757 119.975) (width 0.4) (layer "B.Cu") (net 2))
 (segment (start 123.825 101.972793) (end 120.2 105.597793) (width 0.4) (layer "B.Cu") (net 2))
 (segment (start 119.2 85.725) (end 126.275 85.725) (width 0.4) (layer "B.Cu") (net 2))
 (segment (start 120.2 114.418) (end 123.441 117.659) (width 0.4) (layer "B.Cu") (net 2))
 (segment (start 122.8535 117.0715) (end 125.5 114.425) (width 0.4) (layer "B.Cu") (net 2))
 (segment (start 122.5875 96.9625) (end 123.325 96.225) (width 0.4) (layer "B.Cu") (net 2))
 (segment (start 127.7 98.6975) (end 127.7 97.78) (width 0.2) (layer "F.Cu") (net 15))
 (segment (start 129.942 100.9395) (end 127.7 98.6975) (width 0.2) (layer "F.Cu") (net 15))
 (segment (start 128.2 101.7375) (end 128.2 100.675) (width 0.2) (layer "F.Cu") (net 16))
 (segment (start 127.05 99.525) (end 127.05 97.78) (width 0.2) (layer "F.Cu") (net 16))
 (segment (start 128.2 100.675) (end 127.05 99.525) (width 0.2) (layer "F.Cu") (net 16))
 (segment (start 129.942 103.4795) (end 128.2 101.7375) (width 0.2) (layer "F.Cu") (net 16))
 (segment (start 126.585501 93.3195) (end 126.43 93.475001) (width 0.2) (layer "F.Cu") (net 9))
 (segment (start 126.43 93.475001) (end 126.43 97.75) (width 0.2) (layer "F.Cu") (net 9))
 (segment (start 126.43 97.75) (end 126.4 97.78) (width 0.2) (layer "F.Cu") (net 9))
 (segment (start 129.942 93.3195) (end 126.585501 93.3195) (width 0.2) (layer "F.Cu") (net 9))
 (segment (start 125.775 96.3) (end 125.775 97.755) (width 0.2) (layer "F.Cu") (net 4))
 (segment (start 122.288629 95.875) (end 122.951371 95.875) (width 0.2) (layer "F.Cu") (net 4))
 (segment (start 120.712451 89.700001) (end 120.712451 95.062451) (width 0.2) (layer "F.Cu") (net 4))
 (segment (start 122.213629 95.8) (end 122.288629 95.875) (width 0.2) (layer "F.Cu") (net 4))
 (segment (start 122.951371 95.875) (end 123.026371 95.8) (width 0.2) (layer "F.Cu") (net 4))
 (segment (start 125.775 97.755) (end 125.75 97.78) (width 0.2) (layer "F.Cu") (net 4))
 (segment (start 120.712451 95.062451) (end 121.45 95.8) (width 0.2) (layer "F.Cu") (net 4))
 (segment (start 121.45 95.8) (end 122.213629 95.8) (width 0.2) (layer "F.Cu") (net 4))
 (segment (start 125.275 95.8) (end 125.775 96.3) (width 0.2) (layer "F.Cu") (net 4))
 (segment (start 123.026371 95.8) (end 125.275 95.8) (width 0.2) (layer "F.Cu") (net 4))
 (segment (start 121.0656 96.500001) (end 124.572256 96.500001) (width 0.2) (layer "F.Cu") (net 3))
 (segment (start 125.1 97.027745) (end 125.1 97.78) (width 0.2) (layer "F.Cu") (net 3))
 (segment (start 124.572256 96.500001) (end 125.1 97.027745) (width 0.2) (layer "F.Cu") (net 3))
 (segment (start 123.825 103.545) (end 123.8 103.52) (width 0.2) (layer "F.Cu") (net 18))
 (segment (start 123.825 105.5) (end 123.825 103.545) (width 0.2) (layer "F.Cu") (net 18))
 (via (at 123.825 105.5) (size 0.6) (drill 0.3) (layers "F.Cu" "B.Cu") (free) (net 18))
 (segment (start 123.825 105.5) (end 126.8845 108.5595) (width 0.2) (layer "B.Cu") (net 18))
 (segment (start 126.8845 108.5595) (end 129.942 108.5595) (width 0.2) (layer "B.Cu") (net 18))
 (segment (start 125.525 108.1644) (end 127.05 106.6394) (width 0.4) (layer "F.Cu") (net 23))
 (segment (start 127.05 106.6394) (end 127.05 103.52) (width 0.4) (layer "F.Cu") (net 23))
 (segment (start 125.525 108.6724) (end 125.525 108.1644) (width 0.4) (layer "F.Cu") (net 23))
 (segment (start 120.712451 87.799999) (end 120.712451 84.687549) (width 0.5) (layer "F.Cu") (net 5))
 (segment (start 122.5 82.9) (end 122.5 81.18) (width 0.5) (layer "F.Cu") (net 5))
 (segment (start 120.712451 84.687549) (end 122.5 82.9) (width 0.5) (layer "F.Cu") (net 5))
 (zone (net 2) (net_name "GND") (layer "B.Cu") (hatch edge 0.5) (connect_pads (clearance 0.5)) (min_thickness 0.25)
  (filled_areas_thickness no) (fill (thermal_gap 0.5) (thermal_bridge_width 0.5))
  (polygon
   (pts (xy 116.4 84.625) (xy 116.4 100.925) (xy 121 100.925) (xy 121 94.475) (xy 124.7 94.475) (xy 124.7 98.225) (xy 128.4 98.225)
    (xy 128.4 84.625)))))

